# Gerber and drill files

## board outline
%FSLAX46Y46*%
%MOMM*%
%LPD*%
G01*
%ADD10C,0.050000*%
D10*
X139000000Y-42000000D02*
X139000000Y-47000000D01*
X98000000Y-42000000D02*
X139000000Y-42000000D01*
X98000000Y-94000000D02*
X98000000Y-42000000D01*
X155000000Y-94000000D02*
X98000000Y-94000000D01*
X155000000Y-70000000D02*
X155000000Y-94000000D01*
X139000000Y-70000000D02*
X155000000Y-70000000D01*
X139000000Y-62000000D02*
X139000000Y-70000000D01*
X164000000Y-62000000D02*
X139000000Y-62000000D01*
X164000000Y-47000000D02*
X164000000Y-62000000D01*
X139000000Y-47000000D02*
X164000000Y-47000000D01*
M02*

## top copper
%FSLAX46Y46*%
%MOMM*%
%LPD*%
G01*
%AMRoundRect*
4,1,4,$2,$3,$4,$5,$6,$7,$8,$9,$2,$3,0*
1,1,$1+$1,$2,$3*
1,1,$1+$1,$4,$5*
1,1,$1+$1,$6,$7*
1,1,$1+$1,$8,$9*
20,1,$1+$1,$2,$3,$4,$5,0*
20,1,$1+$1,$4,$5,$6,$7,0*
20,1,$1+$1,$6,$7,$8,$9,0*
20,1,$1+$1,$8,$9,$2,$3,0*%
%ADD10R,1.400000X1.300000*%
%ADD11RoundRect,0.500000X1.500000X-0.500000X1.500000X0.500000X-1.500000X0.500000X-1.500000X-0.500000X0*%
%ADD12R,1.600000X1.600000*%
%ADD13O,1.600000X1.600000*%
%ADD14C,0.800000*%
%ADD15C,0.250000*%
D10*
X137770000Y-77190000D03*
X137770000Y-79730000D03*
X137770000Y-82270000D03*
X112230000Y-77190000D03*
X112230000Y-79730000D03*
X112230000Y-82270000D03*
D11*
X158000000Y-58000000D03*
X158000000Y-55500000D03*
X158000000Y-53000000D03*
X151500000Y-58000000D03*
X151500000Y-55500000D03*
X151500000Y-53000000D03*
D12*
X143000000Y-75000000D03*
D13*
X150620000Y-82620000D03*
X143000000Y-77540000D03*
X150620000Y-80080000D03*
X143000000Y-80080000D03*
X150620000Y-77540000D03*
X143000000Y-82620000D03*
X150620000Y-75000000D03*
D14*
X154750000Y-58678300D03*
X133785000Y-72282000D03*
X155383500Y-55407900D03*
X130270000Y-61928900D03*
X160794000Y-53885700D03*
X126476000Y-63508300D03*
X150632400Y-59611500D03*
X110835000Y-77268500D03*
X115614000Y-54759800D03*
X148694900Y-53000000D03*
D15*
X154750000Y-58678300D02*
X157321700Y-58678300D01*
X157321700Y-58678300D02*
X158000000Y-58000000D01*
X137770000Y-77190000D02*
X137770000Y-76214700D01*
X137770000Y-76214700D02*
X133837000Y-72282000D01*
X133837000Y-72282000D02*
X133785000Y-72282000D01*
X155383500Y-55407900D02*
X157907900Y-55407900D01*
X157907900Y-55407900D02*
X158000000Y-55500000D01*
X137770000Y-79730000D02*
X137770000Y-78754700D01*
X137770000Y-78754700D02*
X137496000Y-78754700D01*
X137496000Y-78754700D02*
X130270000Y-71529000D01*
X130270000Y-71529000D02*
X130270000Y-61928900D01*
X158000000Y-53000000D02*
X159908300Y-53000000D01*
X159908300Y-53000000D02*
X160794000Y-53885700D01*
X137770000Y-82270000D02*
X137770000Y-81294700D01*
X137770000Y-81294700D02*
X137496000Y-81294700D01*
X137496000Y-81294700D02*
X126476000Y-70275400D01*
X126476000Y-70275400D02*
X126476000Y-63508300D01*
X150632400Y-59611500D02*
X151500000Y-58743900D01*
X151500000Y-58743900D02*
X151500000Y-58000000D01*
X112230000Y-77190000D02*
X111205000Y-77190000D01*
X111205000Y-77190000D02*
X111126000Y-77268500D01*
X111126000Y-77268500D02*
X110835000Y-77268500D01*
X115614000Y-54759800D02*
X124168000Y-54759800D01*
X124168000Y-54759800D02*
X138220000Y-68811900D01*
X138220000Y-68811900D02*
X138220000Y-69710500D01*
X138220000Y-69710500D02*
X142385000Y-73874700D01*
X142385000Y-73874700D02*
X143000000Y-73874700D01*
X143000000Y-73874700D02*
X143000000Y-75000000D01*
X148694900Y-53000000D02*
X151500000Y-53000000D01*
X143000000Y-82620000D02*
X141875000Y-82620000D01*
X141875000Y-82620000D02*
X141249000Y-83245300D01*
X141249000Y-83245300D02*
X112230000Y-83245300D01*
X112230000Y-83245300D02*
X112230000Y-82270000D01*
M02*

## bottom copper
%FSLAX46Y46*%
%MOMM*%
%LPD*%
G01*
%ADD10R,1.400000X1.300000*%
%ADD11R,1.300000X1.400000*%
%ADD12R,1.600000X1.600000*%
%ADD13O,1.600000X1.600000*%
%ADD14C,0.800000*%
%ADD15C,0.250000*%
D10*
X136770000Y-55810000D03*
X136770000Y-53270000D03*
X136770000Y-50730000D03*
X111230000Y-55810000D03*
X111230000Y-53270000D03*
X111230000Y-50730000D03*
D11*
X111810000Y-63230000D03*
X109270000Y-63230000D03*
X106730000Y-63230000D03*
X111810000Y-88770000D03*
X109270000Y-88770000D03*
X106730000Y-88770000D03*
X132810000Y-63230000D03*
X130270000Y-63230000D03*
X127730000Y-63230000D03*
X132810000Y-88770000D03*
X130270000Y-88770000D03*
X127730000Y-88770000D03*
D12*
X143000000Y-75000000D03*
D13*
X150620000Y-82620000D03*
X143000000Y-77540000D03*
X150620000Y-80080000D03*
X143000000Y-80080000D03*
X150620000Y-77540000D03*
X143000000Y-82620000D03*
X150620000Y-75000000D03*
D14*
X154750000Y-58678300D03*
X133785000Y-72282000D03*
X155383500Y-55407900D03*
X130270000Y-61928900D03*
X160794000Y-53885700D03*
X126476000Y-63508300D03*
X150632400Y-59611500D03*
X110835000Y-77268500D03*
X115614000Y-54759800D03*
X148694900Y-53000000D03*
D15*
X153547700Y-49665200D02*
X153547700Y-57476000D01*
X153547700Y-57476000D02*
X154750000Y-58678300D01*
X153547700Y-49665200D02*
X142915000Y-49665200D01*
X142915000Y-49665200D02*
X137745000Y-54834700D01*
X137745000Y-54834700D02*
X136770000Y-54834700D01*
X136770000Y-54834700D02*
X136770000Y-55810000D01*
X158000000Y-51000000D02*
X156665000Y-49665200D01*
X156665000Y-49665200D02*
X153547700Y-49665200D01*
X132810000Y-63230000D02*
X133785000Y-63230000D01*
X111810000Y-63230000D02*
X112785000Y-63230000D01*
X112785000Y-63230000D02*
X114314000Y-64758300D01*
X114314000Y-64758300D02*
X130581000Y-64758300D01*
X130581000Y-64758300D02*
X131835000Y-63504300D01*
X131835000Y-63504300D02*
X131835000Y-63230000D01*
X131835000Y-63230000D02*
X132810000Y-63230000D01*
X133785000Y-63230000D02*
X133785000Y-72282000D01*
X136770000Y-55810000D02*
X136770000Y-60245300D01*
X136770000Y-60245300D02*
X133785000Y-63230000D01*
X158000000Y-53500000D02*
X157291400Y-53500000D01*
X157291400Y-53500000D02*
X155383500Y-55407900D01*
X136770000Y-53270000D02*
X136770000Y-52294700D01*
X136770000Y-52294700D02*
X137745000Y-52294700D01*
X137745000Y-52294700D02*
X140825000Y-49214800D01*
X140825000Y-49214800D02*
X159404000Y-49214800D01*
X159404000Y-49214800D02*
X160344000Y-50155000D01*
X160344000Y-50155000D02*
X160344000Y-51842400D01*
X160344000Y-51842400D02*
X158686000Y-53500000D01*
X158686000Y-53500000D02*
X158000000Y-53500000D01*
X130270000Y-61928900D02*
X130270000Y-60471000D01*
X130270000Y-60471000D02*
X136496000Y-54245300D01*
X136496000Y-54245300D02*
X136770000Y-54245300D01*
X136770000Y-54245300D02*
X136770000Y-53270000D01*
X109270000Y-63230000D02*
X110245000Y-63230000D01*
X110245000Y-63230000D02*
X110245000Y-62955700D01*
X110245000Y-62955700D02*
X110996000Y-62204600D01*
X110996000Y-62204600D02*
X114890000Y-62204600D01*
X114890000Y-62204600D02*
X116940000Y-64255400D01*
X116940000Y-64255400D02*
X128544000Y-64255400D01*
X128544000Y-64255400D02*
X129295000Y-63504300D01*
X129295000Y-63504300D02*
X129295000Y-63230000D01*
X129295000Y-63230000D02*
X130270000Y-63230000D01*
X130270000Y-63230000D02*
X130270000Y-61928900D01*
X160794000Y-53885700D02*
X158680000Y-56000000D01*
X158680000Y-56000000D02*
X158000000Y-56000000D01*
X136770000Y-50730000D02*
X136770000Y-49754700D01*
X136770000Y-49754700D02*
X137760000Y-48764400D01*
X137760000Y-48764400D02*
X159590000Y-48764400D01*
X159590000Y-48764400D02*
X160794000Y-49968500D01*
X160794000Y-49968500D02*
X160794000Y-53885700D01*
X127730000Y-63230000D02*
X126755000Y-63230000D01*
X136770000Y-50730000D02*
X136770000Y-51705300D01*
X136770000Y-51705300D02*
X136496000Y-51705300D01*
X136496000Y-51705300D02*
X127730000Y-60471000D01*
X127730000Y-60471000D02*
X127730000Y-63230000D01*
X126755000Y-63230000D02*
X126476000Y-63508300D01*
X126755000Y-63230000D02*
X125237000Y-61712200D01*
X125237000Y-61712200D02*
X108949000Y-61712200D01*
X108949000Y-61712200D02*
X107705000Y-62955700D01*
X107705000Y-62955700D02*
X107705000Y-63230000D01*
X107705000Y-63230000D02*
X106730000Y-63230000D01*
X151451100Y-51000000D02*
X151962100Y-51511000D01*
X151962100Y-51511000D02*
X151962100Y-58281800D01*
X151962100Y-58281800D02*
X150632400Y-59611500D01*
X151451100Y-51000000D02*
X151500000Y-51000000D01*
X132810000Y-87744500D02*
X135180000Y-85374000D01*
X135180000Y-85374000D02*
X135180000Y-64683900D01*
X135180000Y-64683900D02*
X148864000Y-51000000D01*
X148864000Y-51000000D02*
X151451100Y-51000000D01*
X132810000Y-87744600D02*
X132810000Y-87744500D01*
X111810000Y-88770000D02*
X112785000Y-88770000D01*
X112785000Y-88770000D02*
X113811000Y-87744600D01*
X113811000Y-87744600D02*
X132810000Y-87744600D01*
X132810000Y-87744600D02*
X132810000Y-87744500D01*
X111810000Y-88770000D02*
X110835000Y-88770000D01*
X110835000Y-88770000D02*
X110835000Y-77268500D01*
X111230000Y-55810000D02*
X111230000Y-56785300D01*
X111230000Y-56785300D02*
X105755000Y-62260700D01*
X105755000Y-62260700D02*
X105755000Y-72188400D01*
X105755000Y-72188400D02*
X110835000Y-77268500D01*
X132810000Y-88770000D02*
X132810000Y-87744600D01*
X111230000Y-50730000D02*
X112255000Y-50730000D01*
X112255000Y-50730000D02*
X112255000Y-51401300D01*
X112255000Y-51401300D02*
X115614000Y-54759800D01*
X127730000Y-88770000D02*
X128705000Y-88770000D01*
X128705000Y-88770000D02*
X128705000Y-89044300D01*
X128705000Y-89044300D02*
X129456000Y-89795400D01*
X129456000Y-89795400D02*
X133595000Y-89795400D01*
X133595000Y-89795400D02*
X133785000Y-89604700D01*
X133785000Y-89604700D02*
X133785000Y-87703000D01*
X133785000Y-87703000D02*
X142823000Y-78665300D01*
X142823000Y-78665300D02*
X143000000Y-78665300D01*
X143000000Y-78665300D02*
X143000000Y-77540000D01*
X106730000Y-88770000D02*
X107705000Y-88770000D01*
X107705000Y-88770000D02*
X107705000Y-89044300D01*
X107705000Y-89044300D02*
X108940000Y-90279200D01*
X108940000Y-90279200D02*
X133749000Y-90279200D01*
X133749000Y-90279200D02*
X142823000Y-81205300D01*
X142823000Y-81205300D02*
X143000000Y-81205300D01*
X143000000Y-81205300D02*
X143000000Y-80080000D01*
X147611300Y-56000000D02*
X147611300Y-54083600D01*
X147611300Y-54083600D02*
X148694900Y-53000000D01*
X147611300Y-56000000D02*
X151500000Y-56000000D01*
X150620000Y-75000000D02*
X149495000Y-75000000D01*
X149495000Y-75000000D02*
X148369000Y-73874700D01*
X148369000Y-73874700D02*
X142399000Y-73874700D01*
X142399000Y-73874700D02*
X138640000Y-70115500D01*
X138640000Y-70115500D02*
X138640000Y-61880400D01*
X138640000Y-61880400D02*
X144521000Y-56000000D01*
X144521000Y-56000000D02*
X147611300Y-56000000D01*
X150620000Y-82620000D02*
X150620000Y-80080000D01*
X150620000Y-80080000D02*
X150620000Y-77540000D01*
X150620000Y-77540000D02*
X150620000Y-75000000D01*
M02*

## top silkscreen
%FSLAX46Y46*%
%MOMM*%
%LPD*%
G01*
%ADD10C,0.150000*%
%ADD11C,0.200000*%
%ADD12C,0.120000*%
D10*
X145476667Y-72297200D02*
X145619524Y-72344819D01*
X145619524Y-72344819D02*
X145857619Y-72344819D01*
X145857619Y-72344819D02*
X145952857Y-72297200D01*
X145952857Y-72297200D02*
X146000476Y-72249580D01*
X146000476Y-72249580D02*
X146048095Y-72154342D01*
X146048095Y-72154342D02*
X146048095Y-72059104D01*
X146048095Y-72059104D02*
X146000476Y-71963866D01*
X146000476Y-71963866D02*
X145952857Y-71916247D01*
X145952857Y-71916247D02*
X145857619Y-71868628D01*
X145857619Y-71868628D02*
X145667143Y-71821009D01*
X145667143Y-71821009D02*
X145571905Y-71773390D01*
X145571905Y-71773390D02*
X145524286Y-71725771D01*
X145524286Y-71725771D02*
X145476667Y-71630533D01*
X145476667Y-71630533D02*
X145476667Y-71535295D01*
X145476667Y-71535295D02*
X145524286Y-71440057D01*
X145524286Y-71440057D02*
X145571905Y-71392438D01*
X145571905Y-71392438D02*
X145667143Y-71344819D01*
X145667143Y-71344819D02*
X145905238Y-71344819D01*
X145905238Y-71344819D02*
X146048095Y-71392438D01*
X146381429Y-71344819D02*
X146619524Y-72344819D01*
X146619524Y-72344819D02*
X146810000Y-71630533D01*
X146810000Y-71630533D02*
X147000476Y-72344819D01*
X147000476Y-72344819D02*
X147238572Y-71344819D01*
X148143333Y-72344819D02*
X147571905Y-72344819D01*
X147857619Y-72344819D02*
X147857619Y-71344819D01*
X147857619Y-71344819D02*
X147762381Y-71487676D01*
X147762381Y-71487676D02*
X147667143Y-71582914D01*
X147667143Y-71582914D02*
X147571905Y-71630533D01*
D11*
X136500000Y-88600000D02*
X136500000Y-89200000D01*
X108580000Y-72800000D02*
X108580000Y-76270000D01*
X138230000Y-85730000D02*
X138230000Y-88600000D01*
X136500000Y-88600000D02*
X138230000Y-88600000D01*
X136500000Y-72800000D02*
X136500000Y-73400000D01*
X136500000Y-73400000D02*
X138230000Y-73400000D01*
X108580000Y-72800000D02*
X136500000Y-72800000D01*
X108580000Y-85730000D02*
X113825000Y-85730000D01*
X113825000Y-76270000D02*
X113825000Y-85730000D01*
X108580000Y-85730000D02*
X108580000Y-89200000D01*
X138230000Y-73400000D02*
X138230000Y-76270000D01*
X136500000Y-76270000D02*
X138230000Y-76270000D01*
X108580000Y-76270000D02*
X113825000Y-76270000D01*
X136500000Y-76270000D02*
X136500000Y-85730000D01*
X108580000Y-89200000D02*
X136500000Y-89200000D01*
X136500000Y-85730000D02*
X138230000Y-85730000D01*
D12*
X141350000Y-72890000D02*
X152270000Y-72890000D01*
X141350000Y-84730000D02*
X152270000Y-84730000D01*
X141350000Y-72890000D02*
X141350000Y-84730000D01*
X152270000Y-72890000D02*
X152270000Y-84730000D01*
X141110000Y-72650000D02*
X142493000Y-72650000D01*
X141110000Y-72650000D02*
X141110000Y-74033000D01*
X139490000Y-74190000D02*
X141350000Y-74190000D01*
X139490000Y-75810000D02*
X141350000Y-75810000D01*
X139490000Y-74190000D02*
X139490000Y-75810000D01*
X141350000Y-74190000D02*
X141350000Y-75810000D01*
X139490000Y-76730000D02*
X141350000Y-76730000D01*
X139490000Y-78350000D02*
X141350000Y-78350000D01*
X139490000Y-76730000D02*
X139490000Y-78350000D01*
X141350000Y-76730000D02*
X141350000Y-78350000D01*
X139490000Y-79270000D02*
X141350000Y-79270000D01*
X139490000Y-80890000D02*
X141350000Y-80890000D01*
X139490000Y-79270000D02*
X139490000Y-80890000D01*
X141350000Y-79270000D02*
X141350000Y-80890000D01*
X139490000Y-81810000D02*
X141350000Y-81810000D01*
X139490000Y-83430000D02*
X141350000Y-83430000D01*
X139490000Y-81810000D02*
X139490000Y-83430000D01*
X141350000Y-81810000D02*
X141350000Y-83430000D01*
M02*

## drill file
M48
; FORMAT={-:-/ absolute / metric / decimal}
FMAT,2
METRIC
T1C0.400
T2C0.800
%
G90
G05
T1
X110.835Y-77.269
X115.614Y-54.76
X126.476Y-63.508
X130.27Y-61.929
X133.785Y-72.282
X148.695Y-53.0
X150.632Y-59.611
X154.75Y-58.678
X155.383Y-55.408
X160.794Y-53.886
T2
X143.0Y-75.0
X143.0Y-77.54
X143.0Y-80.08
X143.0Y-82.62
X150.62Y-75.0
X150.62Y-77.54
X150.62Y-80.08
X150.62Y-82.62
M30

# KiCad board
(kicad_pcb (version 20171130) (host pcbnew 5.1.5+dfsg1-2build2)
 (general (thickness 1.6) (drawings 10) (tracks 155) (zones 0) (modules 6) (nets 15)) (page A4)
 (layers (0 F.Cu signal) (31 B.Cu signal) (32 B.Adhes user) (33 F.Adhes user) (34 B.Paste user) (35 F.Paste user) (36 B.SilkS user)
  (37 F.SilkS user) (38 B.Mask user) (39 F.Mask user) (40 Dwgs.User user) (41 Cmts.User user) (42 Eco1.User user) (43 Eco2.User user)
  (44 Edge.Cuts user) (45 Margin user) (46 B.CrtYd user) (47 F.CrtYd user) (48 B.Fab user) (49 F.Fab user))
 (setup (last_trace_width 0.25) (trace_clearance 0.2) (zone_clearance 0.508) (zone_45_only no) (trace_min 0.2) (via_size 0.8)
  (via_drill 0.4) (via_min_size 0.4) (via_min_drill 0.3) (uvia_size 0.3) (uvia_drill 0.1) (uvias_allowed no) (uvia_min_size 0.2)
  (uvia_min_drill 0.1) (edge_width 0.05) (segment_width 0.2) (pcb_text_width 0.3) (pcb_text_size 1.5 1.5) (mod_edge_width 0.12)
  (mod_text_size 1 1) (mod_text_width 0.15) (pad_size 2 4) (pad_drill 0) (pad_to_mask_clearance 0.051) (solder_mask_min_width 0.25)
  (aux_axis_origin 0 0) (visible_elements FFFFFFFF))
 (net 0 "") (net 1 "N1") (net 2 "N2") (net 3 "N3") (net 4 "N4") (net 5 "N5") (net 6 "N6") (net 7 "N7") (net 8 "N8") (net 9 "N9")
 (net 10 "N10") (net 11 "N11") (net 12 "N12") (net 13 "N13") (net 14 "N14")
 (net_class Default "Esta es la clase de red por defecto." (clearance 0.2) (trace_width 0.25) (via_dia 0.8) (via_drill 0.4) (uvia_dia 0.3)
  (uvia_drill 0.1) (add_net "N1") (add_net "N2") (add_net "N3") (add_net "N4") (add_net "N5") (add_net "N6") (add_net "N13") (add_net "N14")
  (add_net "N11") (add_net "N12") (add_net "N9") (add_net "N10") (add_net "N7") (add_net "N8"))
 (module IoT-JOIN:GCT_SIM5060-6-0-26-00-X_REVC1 (layer B.Cu) (at 124 52 90)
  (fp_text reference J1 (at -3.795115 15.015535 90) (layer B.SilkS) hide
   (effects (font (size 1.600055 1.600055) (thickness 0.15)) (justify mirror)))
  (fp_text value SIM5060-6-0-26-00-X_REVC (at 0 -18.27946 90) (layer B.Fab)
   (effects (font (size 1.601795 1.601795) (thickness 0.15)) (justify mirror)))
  (pad C1 smd rect (at -3.81 12.77 90) (size 1.3 1.4) (layers B.Cu B.Paste B.Mask) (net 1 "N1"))
  (pad C2 smd rect (at -1.27 12.77 90) (size 1.3 1.4) (layers B.Cu B.Paste B.Mask) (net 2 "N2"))
  (pad C3 smd rect (at 1.27 12.77 90) (size 1.3 1.4) (layers B.Cu B.Paste B.Mask) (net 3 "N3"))
  (pad C5 smd rect (at -3.81 -12.77 90) (size 1.3 1.4) (layers B.Cu B.Paste B.Mask) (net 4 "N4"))
  (pad C6 smd rect (at -1.27 -12.77 90) (size 1.3 1.4) (layers B.Cu B.Paste B.Mask) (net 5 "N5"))
  (pad C7 smd rect (at 1.27 -12.77 90) (size 1.3 1.4) (layers B.Cu B.Paste B.Mask) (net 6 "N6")))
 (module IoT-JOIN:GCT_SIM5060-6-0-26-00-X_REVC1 (layer F.Cu) (at 125 81 270)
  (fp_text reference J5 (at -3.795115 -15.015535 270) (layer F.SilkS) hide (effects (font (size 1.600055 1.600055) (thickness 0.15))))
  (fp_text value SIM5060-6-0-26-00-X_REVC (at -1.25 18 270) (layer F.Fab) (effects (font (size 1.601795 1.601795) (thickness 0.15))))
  (fp_line (start 7.6 -11.5) (end 8.2 -11.5) (layer F.SilkS) (width 0.2))
  (fp_line (start -8.2 16.42) (end -4.73 16.42) (layer F.SilkS) (width 0.2))
  (fp_line (start 4.73 -13.23) (end 7.6 -13.23) (layer F.SilkS) (width 0.2))
  (fp_line (start 7.6 -11.5) (end 7.6 -13.23) (layer F.SilkS) (width 0.2))
  (fp_line (start -8.2 -11.5) (end -7.6 -11.5) (layer F.SilkS) (width 0.2))
  (fp_line (start -7.6 -11.5) (end -7.6 -13.23) (layer F.SilkS) (width 0.2))
  (fp_line (start -8.2 16.42) (end -8.2 -11.5) (layer F.SilkS) (width 0.2))
  (fp_line (start 4.73 16.42) (end 4.73 11.175) (layer F.SilkS) (width 0.2))
  (fp_line (start -4.73 11.175) (end 4.73 11.175) (layer F.SilkS) (width 0.2))
  (fp_line (start 4.73 16.42) (end 8.2 16.42) (layer F.SilkS) (width 0.2))
  (fp_line (start -7.6 -13.23) (end -4.73 -13.23) (layer F.SilkS) (width 0.2))
  (fp_line (start -4.73 -11.5) (end -4.73 -13.23) (layer F.SilkS) (width 0.2))
  (fp_line (start -4.73 16.42) (end -4.73 11.175) (layer F.SilkS) (width 0.2))
  (fp_line (start -4.73 -11.5) (end 4.73 -11.5) (layer F.SilkS) (width 0.2))
  (fp_line (start 8.2 16.42) (end 8.2 -11.5) (layer F.SilkS) (width 0.2))
  (fp_line (start 4.73 -11.5) (end 4.73 -13.23) (layer F.SilkS) (width 0.2))
  (pad C1 smd rect (at -3.81 -12.77 270) (size 1.3 1.4) (layers F.Cu F.Paste F.Mask) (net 1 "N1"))
  (pad C2 smd rect (at -1.27 -12.77 270) (size 1.3 1.4) (layers F.Cu F.Paste F.Mask) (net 2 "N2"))
  (pad C3 smd rect (at 1.27 -12.77 270) (size 1.3 1.4) (layers F.Cu F.Paste F.Mask) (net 3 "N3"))
  (pad C5 smd rect (at -3.81 12.77 270) (size 1.3 1.4) (layers F.Cu F.Paste F.Mask) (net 4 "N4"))
  (pad C6 smd rect (at -1.27 12.77 270) (size 1.3 1.4) (layers F.Cu F.Paste F.Mask) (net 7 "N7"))
  (pad C7 smd rect (at 1.27 12.77 270) (size 1.3 1.4) (layers F.Cu F.Paste F.Mask) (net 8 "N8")))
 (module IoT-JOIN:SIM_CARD (layer F.Cu) (at 164 62 90)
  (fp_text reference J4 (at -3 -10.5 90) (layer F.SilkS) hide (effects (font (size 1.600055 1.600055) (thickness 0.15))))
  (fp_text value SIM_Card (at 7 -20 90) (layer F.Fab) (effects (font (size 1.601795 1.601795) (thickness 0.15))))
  (pad 1 connect roundrect (at 4 -6 90) (size 2 4) (layers F.Cu F.Mask) (roundrect_rratio 0.25) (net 1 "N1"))
  (pad 2 connect roundrect (at 6.5 -6 90) (size 2 4) (layers F.Cu F.Mask) (roundrect_rratio 0.25) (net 2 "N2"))
  (pad 3 connect roundrect (at 9 -6 90) (size 2 4) (layers F.Cu F.Mask) (roundrect_rratio 0.25) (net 3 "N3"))
  (pad 5 connect roundrect (at 4 -12.5 90) (size 2 4) (layers F.Cu F.Mask) (roundrect_rratio 0.25) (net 4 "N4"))
  (pad 6 connect roundrect (at 6.5 -12.5 90) (size 2 4) (layers F.Cu F.Mask) (roundrect_rratio 0.25) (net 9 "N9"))
  (pad 7 connect roundrect (at 9 -12.5 90) (size 2 4) (layers F.Cu F.Mask) (roundrect_rratio 0.25) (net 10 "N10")))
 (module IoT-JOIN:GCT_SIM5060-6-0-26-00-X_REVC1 (layer B.Cu) (at 108 76 180)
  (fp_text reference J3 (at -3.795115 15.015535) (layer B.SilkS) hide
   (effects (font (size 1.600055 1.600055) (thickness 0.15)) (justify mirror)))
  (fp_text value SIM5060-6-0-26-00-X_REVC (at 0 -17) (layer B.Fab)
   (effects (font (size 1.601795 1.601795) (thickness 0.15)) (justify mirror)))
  (pad C1 smd rect (at -3.81 12.77 180) (size 1.3 1.4) (layers B.Cu B.Paste B.Mask) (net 1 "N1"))
  (pad C2 smd rect (at -1.27 12.77 180) (size 1.3 1.4) (layers B.Cu B.Paste B.Mask) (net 2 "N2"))
  (pad C3 smd rect (at 1.27 12.77 180) (size 1.3 1.4) (layers B.Cu B.Paste B.Mask) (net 3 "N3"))
  (pad C5 smd rect (at -3.81 -12.77 180) (size 1.3 1.4) (layers B.Cu B.Paste B.Mask) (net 4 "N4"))
  (pad C6 smd rect (at -1.27 -12.77 180) (size 1.3 1.4) (layers B.Cu B.Paste B.Mask) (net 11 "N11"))
  (pad C7 smd rect (at 1.27 -12.77 180) (size 1.3 1.4) (layers B.Cu B.Paste B.Mask) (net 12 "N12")))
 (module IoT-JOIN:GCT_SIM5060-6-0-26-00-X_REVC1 (layer B.Cu) (at 129 76 180)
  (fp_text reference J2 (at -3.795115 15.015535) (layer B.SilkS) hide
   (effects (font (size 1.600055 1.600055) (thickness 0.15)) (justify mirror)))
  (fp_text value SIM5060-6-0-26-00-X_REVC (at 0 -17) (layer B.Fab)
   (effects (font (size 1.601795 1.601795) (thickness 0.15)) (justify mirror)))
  (pad C1 smd rect (at -3.81 12.77 180) (size 1.3 1.4) (layers B.Cu B.Paste B.Mask) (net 1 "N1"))
  (pad C2 smd rect (at -1.27 12.77 180) (size 1.3 1.4) (layers B.Cu B.Paste B.Mask) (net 2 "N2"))
  (pad C3 smd rect (at 1.27 12.77 180) (size 1.3 1.4) (layers B.Cu B.Paste B.Mask) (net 3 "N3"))
  (pad C5 smd rect (at -3.81 -12.77 180) (size 1.3 1.4) (layers B.Cu B.Paste B.Mask) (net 4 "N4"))
  (pad C6 smd rect (at -1.27 -12.77 180) (size 1.3 1.4) (layers B.Cu B.Paste B.Mask) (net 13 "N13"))
  (pad C7 smd rect (at 1.27 -12.77 180) (size 1.3 1.4) (layers B.Cu B.Paste B.Mask) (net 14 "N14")))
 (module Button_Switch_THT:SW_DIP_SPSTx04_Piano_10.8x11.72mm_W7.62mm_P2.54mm (layer F.Cu) (at 143 75)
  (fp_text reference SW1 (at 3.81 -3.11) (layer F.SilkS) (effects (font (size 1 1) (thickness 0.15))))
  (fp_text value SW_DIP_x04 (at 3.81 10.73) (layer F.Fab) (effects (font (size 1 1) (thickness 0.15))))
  (fp_line (start -1.65 -2.11) (end 9.27 -2.11) (layer F.SilkS) (width 0.12))
  (fp_line (start -1.65 9.73) (end 9.27 9.73) (layer F.SilkS) (width 0.12))
  (fp_line (start -1.65 -2.11) (end -1.65 9.73) (layer F.SilkS) (width 0.12))
  (fp_line (start 9.27 -2.11) (end 9.27 9.73) (layer F.SilkS) (width 0.12))
  (fp_line (start -1.89 -2.35) (end -0.507 -2.35) (layer F.SilkS) (width 0.12))
  (fp_line (start -1.89 -2.35) (end -1.89 -0.967) (layer F.SilkS) (width 0.12))
  (fp_line (start -3.51 -0.81) (end -1.65 -0.81) (layer F.SilkS) (width 0.12))
  (fp_line (start -3.51 0.81) (end -1.65 0.81) (layer F.SilkS) (width 0.12))
  (fp_line (start -3.51 -0.81) (end -3.51 0.81) (layer F.SilkS) (width 0.12))
  (fp_line (start -1.65 -0.81) (end -1.65 0.81) (layer F.SilkS) (width 0.12))
  (fp_line (start -3.51 1.73) (end -1.65 1.73) (layer F.SilkS) (width 0.12))
  (fp_line (start -3.51 3.35) (end -1.65 3.35) (layer F.SilkS) (width 0.12))
  (fp_line (start -3.51 1.73) (end -3.51 3.35) (layer F.SilkS) (width 0.12))
  (fp_line (start -1.65 1.73) (end -1.65 3.35) (layer F.SilkS) (width 0.12))
  (fp_line (start -3.51 4.27) (end -1.65 4.27) (layer F.SilkS) (width 0.12))
  (fp_line (start -3.51 5.89) (end -1.65 5.89) (layer F.SilkS) (width 0.12))
  (fp_line (start -3.51 4.27) (end -3.51 5.89) (layer F.SilkS) (width 0.12))
  (fp_line (start -1.65 4.27) (end -1.65 5.89) (layer F.SilkS) (width 0.12))
  (fp_line (start -3.51 6.81) (end -1.65 6.81) (layer F.SilkS) (width 0.12))
  (fp_line (start -3.51 8.43) (end -1.65 8.43) (layer F.SilkS) (width 0.12))
  (fp_line (start -3.51 6.81) (end -3.51 8.43) (layer F.SilkS) (width 0.12))
  (fp_line (start -1.65 6.81) (end -1.65 8.43) (layer F.SilkS) (width 0.12))
  (pad 1 thru_hole rect (at 0 0) (size 1.6 1.6) (drill 0.8) (layers *.Cu *.Mask) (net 6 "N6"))
  (pad 5 thru_hole oval (at 7.62 7.62) (size 1.6 1.6) (drill 0.8) (layers *.Cu *.Mask) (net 10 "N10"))
  (pad 2 thru_hole oval (at 0 2.54) (size 1.6 1.6) (drill 0.8) (layers *.Cu *.Mask) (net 14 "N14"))
  (pad 6 thru_hole oval (at 7.62 5.08) (size 1.6 1.6) (drill 0.8) (layers *.Cu *.Mask) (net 10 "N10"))
  (pad 3 thru_hole oval (at 0 5.08) (size 1.6 1.6) (drill 0.8) (layers *.Cu *.Mask) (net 12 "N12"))
  (pad 7 thru_hole oval (at 7.62 2.54) (size 1.6 1.6) (drill 0.8) (layers *.Cu *.Mask) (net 10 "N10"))
  (pad 4 thru_hole oval (at 0 7.62) (size 1.6 1.6) (drill 0.8) (layers *.Cu *.Mask) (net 8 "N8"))
  (pad 8 thru_hole oval (at 7.62 0) (size 1.6 1.6) (drill 0.8) (layers *.Cu *.Mask) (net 10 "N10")))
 (gr_line (start 139 42) (end 139 47) (layer Edge.Cuts) (width 0.05))
 (gr_line (start 98 42) (end 139 42) (layer Edge.Cuts) (width 0.05))
 (gr_line (start 98 94) (end 98 42) (layer Edge.Cuts) (width 0.05))
 (gr_line (start 155 94) (end 98 94) (layer Edge.Cuts) (width 0.05))
 (gr_line (start 155 70) (end 155 94) (layer Edge.Cuts) (width 0.05))
 (gr_line (start 139 70) (end 155 70) (layer Edge.Cuts) (width 0.05))
 (gr_line (start 139 62) (end 139 70) (layer Edge.Cuts) (width 0.05))
 (gr_line (start 164 62) (end 139 62) (layer Edge.Cuts) (width 0.05))
 (gr_line (start 164 47) (end 164 62) (layer Edge.Cuts) (width 0.05))
 (gr_line (start 139 47) (end 164 47) (layer Edge.Cuts) (width 0.05))
 (segment (start 154.75 58.6783) (end 157.3217 58.6783) (width 0.25) (layer F.Cu) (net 1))
 (segment (start 157.3217 58.6783) (end 158 58) (width 0.25) (layer F.Cu) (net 1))
 (segment (start 153.5477 49.6652) (end 153.5477 57.476) (width 0.25) (layer B.Cu) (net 1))
 (segment (start 153.5477 57.476) (end 154.75 58.6783) (width 0.25) (layer B.Cu) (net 1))
 (segment (start 153.5477 49.6652) (end 142.915 49.6652) (width 0.25) (layer B.Cu) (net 1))
 (segment (start 142.915 49.6652) (end 137.745 54.8347) (width 0.25) (layer B.Cu) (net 1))
 (segment (start 137.745 54.8347) (end 136.77 54.8347) (width 0.25) (layer B.Cu) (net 1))
 (segment (start 136.77 54.8347) (end 136.77 55.81) (width 0.25) (layer B.Cu) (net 1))
 (segment (start 158 51) (end 156.665 49.6652) (width 0.25) (layer B.Cu) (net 1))
 (segment (start 156.665 49.6652) (end 153.5477 49.6652) (width 0.25) (layer B.Cu) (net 1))
 (segment (start 132.81 63.23) (end 133.785 63.23) (width 0.25) (layer B.Cu) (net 1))
 (segment (start 111.81 63.23) (end 112.785 63.23) (width 0.25) (layer B.Cu) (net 1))
 (segment (start 112.785 63.23) (end 114.314 64.7583) (width 0.25) (layer B.Cu) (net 1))
 (segment (start 114.314 64.7583) (end 130.581 64.7583) (width 0.25) (layer B.Cu) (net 1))
 (segment (start 130.581 64.7583) (end 131.835 63.5043) (width 0.25) (layer B.Cu) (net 1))
 (segment (start 131.835 63.5043) (end 131.835 63.23) (width 0.25) (layer B.Cu) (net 1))
 (segment (start 131.835 63.23) (end 132.81 63.23) (width 0.25) (layer B.Cu) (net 1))
 (segment (start 137.77 77.19) (end 137.77 76.2147) (width 0.25) (layer F.Cu) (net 1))
 (segment (start 137.77 76.2147) (end 133.837 72.282) (width 0.25) (layer F.Cu) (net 1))
 (segment (start 133.837 72.282) (end 133.785 72.282) (width 0.25) (layer F.Cu) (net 1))
 (segment (start 133.785 63.23) (end 133.785 72.282) (width 0.25) (layer B.Cu) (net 1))
 (segment (start 136.77 55.81) (end 136.77 60.2453) (width 0.25) (layer B.Cu) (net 1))
 (segment (start 136.77 60.2453) (end 133.785 63.23) (width 0.25) (layer B.Cu) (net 1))
 (via (at 154.75 58.6783) (size 0.8) (layers F.Cu B.Cu) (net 1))
 (via (at 133.785 72.282) (size 0.8) (layers F.Cu B.Cu) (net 1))
 (segment (start 155.3835 55.4079) (end 157.9079 55.4079) (width 0.25) (layer F.Cu) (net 2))
 (segment (start 157.9079 55.4079) (end 158 55.5) (width 0.25) (layer F.Cu) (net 2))
 (segment (start 158 53.5) (end 157.2914 53.5) (width 0.25) (layer B.Cu) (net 2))
 (segment (start 157.2914 53.5) (end 155.3835 55.4079) (width 0.25) (layer B.Cu) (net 2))
 (segment (start 136.77 53.27) (end 136.77 52.2947) (width 0.25) (layer B.Cu) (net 2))
 (segment (start 136.77 52.2947) (end 137.745 52.2947) (width 0.25) (layer B.Cu) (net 2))
 (segment (start 137.745 52.2947) (end 140.825 49.2148) (width 0.25) (layer B.Cu) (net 2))
 (segment (start 140.825 49.2148) (end 159.404 49.2148) (width 0.25) (layer B.Cu) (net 2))
 (segment (start 159.404 49.2148) (end 160.344 50.155) (width 0.25) (layer B.Cu) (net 2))
 (segment (start 160.344 50.155) (end 160.344 51.8424) (width 0.25) (layer B.Cu) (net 2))
 (segment (start 160.344 51.8424) (end 158.686 53.5) (width 0.25) (layer B.Cu) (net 2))
 (segment (start 158.686 53.5) (end 158 53.5) (width 0.25) (layer B.Cu) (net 2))
 (segment (start 137.77 79.73) (end 137.77 78.7547) (width 0.25) (layer F.Cu) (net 2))
 (segment (start 137.77 78.7547) (end 137.496 78.7547) (width 0.25) (layer F.Cu) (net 2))
 (segment (start 137.496 78.7547) (end 130.27 71.529) (width 0.25) (layer F.Cu) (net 2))
 (segment (start 130.27 71.529) (end 130.27 61.9289) (width 0.25) (layer F.Cu) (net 2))
 (segment (start 130.27 61.9289) (end 130.27 60.471) (width 0.25) (layer B.Cu) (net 2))
 (segment (start 130.27 60.471) (end 136.496 54.2453) (width 0.25) (layer B.Cu) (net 2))
 (segment (start 136.496 54.2453) (end 136.77 54.2453) (width 0.25) (layer B.Cu) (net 2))
 (segment (start 136.77 54.2453) (end 136.77 53.27) (width 0.25) (layer B.Cu) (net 2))
 (segment (start 109.27 63.23) (end 110.245 63.23) (width 0.25) (layer B.Cu) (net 2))
 (segment (start 110.245 63.23) (end 110.245 62.9557) (width 0.25) (layer B.Cu) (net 2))
 (segment (start 110.245 62.9557) (end 110.996 62.2046) (width 0.25) (layer B.Cu) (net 2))
 (segment (start 110.996 62.2046) (end 114.89 62.2046) (width 0.25) (layer B.Cu) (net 2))
 (segment (start 114.89 62.2046) (end 116.94 64.2554) (width 0.25) (layer B.Cu) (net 2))
 (segment (start 116.94 64.2554) (end 128.544 64.2554) (width 0.25) (layer B.Cu) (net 2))
 (segment (start 128.544 64.2554) (end 129.295 63.5043) (width 0.25) (layer B.Cu) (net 2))
 (segment (start 129.295 63.5043) (end 129.295 63.23) (width 0.25) (layer B.Cu) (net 2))
 (segment (start 129.295 63.23) (end 130.27 63.23) (width 0.25) (layer B.Cu) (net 2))
 (segment (start 130.27 63.23) (end 130.27 61.9289) (width 0.25) (layer B.Cu) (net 2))
 (via (at 155.3835 55.4079) (size 0.8) (layers F.Cu B.Cu) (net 2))
 (via (at 130.27 61.9289) (size 0.8) (layers F.Cu B.Cu) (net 2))
 (segment (start 158 53) (end 159.9083 53) (width 0.25) (layer F.Cu) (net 3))
 (segment (start 159.9083 53) (end 160.794 53.8857) (width 0.25) (layer F.Cu) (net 3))
 (segment (start 160.794 53.8857) (end 158.68 56) (width 0.25) (layer B.Cu) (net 3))
 (segment (start 158.68 56) (end 158 56) (width 0.25) (layer B.Cu) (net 3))
 (segment (start 136.77 50.73) (end 136.77 49.7547) (width 0.25) (layer B.Cu) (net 3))
 (segment (start 136.77 49.7547) (end 137.76 48.7644) (width 0.25) (layer B.Cu) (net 3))
 (segment (start 137.76 48.7644) (end 159.59 48.7644) (width 0.25) (layer B.Cu) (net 3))
 (segment (start 159.59 48.7644) (end 160.794 49.9685) (width 0.25) (layer B.Cu) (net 3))
 (segment (start 160.794 49.9685) (end 160.794 53.8857) (width 0.25) (layer B.Cu) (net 3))
 (segment (start 127.73 63.23) (end 126.755 63.23) (width 0.25) (layer B.Cu) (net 3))
 (segment (start 136.77 50.73) (end 136.77 51.7053) (width 0.25) (layer B.Cu) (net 3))
 (segment (start 136.77 51.7053) (end 136.496 51.7053) (width 0.25) (layer B.Cu) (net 3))
 (segment (start 136.496 51.7053) (end 127.73 60.471) (width 0.25) (layer B.Cu) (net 3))
 (segment (start 127.73 60.471) (end 127.73 63.23) (width 0.25) (layer B.Cu) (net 3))
 (segment (start 137.77 82.27) (end 137.77 81.2947) (width 0.25) (layer F.Cu) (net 3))
 (segment (start 137.77 81.2947) (end 137.496 81.2947) (width 0.25) (layer F.Cu) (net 3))
 (segment (start 137.496 81.2947) (end 126.476 70.2754) (width 0.25) (layer F.Cu) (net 3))
 (segment (start 126.476 70.2754) (end 126.476 63.5083) (width 0.25) (layer F.Cu) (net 3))
 (segment (start 126.755 63.23) (end 126.476 63.5083) (width 0.25) (layer B.Cu) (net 3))
 (segment (start 126.755 63.23) (end 125.237 61.7122) (width 0.25) (layer B.Cu) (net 3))
 (segment (start 125.237 61.7122) (end 108.949 61.7122) (width 0.25) (layer B.Cu) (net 3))
 (segment (start 108.949 61.7122) (end 107.705 62.9557) (width 0.25) (layer B.Cu) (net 3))
 (segment (start 107.705 62.9557) (end 107.705 63.23) (width 0.25) (layer B.Cu) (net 3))
 (segment (start 107.705 63.23) (end 106.73 63.23) (width 0.25) (layer B.Cu) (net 3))
 (via (at 160.794 53.8857) (size 0.8) (layers F.Cu B.Cu) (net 3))
 (via (at 126.476 63.5083) (size 0.8) (layers F.Cu B.Cu) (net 3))
 (segment (start 150.6324 59.6115) (end 151.5 58.7439) (width 0.25) (layer F.Cu) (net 4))
 (segment (start 151.5 58.7439) (end 151.5 58) (width 0.25) (layer F.Cu) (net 4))
 (segment (start 151.4511 51) (end 151.9621 51.511) (width 0.25) (layer B.Cu) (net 4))
 (segment (start 151.9621 51.511) (end 151.9621 58.2818) (width 0.25) (layer B.Cu) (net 4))
 (segment (start 151.9621 58.2818) (end 150.6324 59.6115) (width 0.25) (layer B.Cu) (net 4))
 (segment (start 151.4511 51) (end 151.5 51) (width 0.25) (layer B.Cu) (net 4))
 (segment (start 132.81 87.7445) (end 135.18 85.374) (width 0.25) (layer B.Cu) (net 4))
 (segment (start 135.18 85.374) (end 135.18 64.6839) (width 0.25) (layer B.Cu) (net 4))
 (segment (start 135.18 64.6839) (end 148.864 51) (width 0.25) (layer B.Cu) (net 4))
 (segment (start 148.864 51) (end 151.4511 51) (width 0.25) (layer B.Cu) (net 4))
 (segment (start 132.81 87.7446) (end 132.81 87.7445) (width 0.25) (layer B.Cu) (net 4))
 (segment (start 111.81 88.77) (end 112.785 88.77) (width 0.25) (layer B.Cu) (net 4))
 (segment (start 112.785 88.77) (end 113.811 87.7446) (width 0.25) (layer B.Cu) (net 4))
 (segment (start 113.811 87.7446) (end 132.81 87.7446) (width 0.25) (layer B.Cu) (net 4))
 (segment (start 132.81 87.7446) (end 132.81 87.7445) (width 0.25) (layer B.Cu) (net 4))
 (segment (start 112.23 77.19) (end 111.205 77.19) (width 0.25) (layer F.Cu) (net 4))
 (segment (start 111.205 77.19) (end 111.126 77.2685) (width 0.25) (layer F.Cu) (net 4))
 (segment (start 111.126 77.2685) (end 110.835 77.2685) (width 0.25) (layer F.Cu) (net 4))
 (segment (start 111.81 88.77) (end 110.835 88.77) (width 0.25) (layer B.Cu) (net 4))
 (segment (start 110.835 88.77) (end 110.835 77.2685) (width 0.25) (layer B.Cu) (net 4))
 (segment (start 111.23 55.81) (end 111.23 56.7853) (width 0.25) (layer B.Cu) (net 4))
 (segment (start 111.23 56.7853) (end 105.755 62.2607) (width 0.25) (layer B.Cu) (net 4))
 (segment (start 105.755 62.2607) (end 105.755 72.1884) (width 0.25) (layer B.Cu) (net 4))
 (segment (start 105.755 72.1884) (end 110.835 77.2685) (width 0.25) (layer B.Cu) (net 4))
 (segment (start 132.81 88.77) (end 132.81 87.7446) (width 0.25) (layer B.Cu) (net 4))
 (via (at 150.6324 59.6115) (size 0.8) (layers F.Cu B.Cu) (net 4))
 (via (at 110.835 77.2685) (size 0.8) (layers F.Cu B.Cu) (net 4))
 (segment (start 111.23 50.73) (end 112.255 50.73) (width 0.25) (layer B.Cu) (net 6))
 (segment (start 112.255 50.73) (end 112.255 51.4013) (width 0.25) (layer B.Cu) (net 6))
 (segment (start 112.255 51.4013) (end 115.614 54.7598) (width 0.25) (layer B.Cu) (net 6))
 (segment (start 115.614 54.7598) (end 124.168 54.7598) (width 0.25) (layer F.Cu) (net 6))
 (segment (start 124.168 54.7598) (end 138.22 68.8119) (width 0.25) (layer F.Cu) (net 6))
 (segment (start 138.22 68.8119) (end 138.22 69.7105) (width 0.25) (layer F.Cu) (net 6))
 (segment (start 138.22 69.7105) (end 142.385 73.8747) (width 0.25) (layer F.Cu) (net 6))
 (segment (start 142.385 73.8747) (end 143 73.8747) (width 0.25) (layer F.Cu) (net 6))
 (segment (start 143 73.8747) (end 143 75) (width 0.25) (layer F.Cu) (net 6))
 (via (at 115.614 54.7598) (size 0.8) (layers F.Cu B.Cu) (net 6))
 (segment (start 127.73 88.77) (end 128.705 88.77) (width 0.25) (layer B.Cu) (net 14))
 (segment (start 128.705 88.77) (end 128.705 89.0443) (width 0.25) (layer B.Cu) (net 14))
 (segment (start 128.705 89.0443) (end 129.456 89.7954) (width 0.25) (layer B.Cu) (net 14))
 (segment (start 129.456 89.7954) (end 133.595 89.7954) (width 0.25) (layer B.Cu) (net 14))
 (segment (start 133.595 89.7954) (end 133.785 89.6047) (width 0.25) (layer B.Cu) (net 14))
 (segment (start 133.785 89.6047) (end 133.785 87.703) (width 0.25) (layer B.Cu) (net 14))
 (segment (start 133.785 87.703) (end 142.823 78.6653) (width 0.25) (layer B.Cu) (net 14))
 (segment (start 142.823 78.6653) (end 143 78.6653) (width 0.25) (layer B.Cu) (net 14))
 (segment (start 143 78.6653) (end 143 77.54) (width 0.25) (layer B.Cu) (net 14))
 (segment (start 106.73 88.77) (end 107.705 88.77) (width 0.25) (layer B.Cu) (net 12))
 (segment (start 107.705 88.77) (end 107.705 89.0443) (width 0.25) (layer B.Cu) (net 12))
 (segment (start 107.705 89.0443) (end 108.94 90.2792) (width 0.25) (layer B.Cu) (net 12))
 (segment (start 108.94 90.2792) (end 133.749 90.2792) (width 0.25) (layer B.Cu) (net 12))
 (segment (start 133.749 90.2792) (end 142.823 81.2053) (width 0.25) (layer B.Cu) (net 12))
 (segment (start 142.823 81.2053) (end 143 81.2053) (width 0.25) (layer B.Cu) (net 12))
 (segment (start 143 81.2053) (end 143 80.08) (width 0.25) (layer B.Cu) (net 12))
 (segment (start 148.6949 53) (end 151.5 53) (width 0.25) (layer F.Cu) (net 10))
 (segment (start 147.6113 56) (end 147.6113 54.0836) (width 0.25) (layer B.Cu) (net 10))
 (segment (start 147.6113 54.0836) (end 148.6949 53) (width 0.25) (layer B.Cu) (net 10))
 (segment (start 147.6113 56) (end 151.5 56) (width 0.25) (layer B.Cu) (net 10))
 (segment (start 150.62 75) (end 149.495 75) (width 0.25) (layer B.Cu) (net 10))
 (segment (start 149.495 75) (end 148.369 73.8747) (width 0.25) (layer B.Cu) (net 10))
 (segment (start 148.369 73.8747) (end 142.399 73.8747) (width 0.25) (layer B.Cu) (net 10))
 (segment (start 142.399 73.8747) (end 138.64 70.1155) (width 0.25) (layer B.Cu) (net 10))
 (segment (start 138.64 70.1155) (end 138.64 61.8804) (width 0.25) (layer B.Cu) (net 10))
 (segment (start 138.64 61.8804) (end 144.521 56) (width 0.25) (layer B.Cu) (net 10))
 (segment (start 144.521 56) (end 147.6113 56) (width 0.25) (layer B.Cu) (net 10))
 (segment (start 150.62 82.62) (end 150.62 80.08) (width 0.25) (layer B.Cu) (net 10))
 (segment (start 150.62 80.08) (end 150.62 77.54) (width 0.25) (layer B.Cu) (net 10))
 (segment (start 150.62 77.54) (end 150.62 75) (width 0.25) (layer B.Cu) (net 10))
 (via (at 148.6949 53) (size 0.8) (layers F.Cu B.Cu) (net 10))
 (segment (start 143 82.62) (end 141.875 82.62) (width 0.25) (layer F.Cu) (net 8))
 (segment (start 141.875 82.62) (end 141.249 83.2453) (width 0.25) (layer F.Cu) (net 8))
 (segment (start 141.249 83.2453) (end 112.23 83.2453) (width 0.25) (layer F.Cu) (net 8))
 (segment (start 112.23 83.2453) (end 112.23 82.27) (width 0.25) (layer F.Cu) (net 8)))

